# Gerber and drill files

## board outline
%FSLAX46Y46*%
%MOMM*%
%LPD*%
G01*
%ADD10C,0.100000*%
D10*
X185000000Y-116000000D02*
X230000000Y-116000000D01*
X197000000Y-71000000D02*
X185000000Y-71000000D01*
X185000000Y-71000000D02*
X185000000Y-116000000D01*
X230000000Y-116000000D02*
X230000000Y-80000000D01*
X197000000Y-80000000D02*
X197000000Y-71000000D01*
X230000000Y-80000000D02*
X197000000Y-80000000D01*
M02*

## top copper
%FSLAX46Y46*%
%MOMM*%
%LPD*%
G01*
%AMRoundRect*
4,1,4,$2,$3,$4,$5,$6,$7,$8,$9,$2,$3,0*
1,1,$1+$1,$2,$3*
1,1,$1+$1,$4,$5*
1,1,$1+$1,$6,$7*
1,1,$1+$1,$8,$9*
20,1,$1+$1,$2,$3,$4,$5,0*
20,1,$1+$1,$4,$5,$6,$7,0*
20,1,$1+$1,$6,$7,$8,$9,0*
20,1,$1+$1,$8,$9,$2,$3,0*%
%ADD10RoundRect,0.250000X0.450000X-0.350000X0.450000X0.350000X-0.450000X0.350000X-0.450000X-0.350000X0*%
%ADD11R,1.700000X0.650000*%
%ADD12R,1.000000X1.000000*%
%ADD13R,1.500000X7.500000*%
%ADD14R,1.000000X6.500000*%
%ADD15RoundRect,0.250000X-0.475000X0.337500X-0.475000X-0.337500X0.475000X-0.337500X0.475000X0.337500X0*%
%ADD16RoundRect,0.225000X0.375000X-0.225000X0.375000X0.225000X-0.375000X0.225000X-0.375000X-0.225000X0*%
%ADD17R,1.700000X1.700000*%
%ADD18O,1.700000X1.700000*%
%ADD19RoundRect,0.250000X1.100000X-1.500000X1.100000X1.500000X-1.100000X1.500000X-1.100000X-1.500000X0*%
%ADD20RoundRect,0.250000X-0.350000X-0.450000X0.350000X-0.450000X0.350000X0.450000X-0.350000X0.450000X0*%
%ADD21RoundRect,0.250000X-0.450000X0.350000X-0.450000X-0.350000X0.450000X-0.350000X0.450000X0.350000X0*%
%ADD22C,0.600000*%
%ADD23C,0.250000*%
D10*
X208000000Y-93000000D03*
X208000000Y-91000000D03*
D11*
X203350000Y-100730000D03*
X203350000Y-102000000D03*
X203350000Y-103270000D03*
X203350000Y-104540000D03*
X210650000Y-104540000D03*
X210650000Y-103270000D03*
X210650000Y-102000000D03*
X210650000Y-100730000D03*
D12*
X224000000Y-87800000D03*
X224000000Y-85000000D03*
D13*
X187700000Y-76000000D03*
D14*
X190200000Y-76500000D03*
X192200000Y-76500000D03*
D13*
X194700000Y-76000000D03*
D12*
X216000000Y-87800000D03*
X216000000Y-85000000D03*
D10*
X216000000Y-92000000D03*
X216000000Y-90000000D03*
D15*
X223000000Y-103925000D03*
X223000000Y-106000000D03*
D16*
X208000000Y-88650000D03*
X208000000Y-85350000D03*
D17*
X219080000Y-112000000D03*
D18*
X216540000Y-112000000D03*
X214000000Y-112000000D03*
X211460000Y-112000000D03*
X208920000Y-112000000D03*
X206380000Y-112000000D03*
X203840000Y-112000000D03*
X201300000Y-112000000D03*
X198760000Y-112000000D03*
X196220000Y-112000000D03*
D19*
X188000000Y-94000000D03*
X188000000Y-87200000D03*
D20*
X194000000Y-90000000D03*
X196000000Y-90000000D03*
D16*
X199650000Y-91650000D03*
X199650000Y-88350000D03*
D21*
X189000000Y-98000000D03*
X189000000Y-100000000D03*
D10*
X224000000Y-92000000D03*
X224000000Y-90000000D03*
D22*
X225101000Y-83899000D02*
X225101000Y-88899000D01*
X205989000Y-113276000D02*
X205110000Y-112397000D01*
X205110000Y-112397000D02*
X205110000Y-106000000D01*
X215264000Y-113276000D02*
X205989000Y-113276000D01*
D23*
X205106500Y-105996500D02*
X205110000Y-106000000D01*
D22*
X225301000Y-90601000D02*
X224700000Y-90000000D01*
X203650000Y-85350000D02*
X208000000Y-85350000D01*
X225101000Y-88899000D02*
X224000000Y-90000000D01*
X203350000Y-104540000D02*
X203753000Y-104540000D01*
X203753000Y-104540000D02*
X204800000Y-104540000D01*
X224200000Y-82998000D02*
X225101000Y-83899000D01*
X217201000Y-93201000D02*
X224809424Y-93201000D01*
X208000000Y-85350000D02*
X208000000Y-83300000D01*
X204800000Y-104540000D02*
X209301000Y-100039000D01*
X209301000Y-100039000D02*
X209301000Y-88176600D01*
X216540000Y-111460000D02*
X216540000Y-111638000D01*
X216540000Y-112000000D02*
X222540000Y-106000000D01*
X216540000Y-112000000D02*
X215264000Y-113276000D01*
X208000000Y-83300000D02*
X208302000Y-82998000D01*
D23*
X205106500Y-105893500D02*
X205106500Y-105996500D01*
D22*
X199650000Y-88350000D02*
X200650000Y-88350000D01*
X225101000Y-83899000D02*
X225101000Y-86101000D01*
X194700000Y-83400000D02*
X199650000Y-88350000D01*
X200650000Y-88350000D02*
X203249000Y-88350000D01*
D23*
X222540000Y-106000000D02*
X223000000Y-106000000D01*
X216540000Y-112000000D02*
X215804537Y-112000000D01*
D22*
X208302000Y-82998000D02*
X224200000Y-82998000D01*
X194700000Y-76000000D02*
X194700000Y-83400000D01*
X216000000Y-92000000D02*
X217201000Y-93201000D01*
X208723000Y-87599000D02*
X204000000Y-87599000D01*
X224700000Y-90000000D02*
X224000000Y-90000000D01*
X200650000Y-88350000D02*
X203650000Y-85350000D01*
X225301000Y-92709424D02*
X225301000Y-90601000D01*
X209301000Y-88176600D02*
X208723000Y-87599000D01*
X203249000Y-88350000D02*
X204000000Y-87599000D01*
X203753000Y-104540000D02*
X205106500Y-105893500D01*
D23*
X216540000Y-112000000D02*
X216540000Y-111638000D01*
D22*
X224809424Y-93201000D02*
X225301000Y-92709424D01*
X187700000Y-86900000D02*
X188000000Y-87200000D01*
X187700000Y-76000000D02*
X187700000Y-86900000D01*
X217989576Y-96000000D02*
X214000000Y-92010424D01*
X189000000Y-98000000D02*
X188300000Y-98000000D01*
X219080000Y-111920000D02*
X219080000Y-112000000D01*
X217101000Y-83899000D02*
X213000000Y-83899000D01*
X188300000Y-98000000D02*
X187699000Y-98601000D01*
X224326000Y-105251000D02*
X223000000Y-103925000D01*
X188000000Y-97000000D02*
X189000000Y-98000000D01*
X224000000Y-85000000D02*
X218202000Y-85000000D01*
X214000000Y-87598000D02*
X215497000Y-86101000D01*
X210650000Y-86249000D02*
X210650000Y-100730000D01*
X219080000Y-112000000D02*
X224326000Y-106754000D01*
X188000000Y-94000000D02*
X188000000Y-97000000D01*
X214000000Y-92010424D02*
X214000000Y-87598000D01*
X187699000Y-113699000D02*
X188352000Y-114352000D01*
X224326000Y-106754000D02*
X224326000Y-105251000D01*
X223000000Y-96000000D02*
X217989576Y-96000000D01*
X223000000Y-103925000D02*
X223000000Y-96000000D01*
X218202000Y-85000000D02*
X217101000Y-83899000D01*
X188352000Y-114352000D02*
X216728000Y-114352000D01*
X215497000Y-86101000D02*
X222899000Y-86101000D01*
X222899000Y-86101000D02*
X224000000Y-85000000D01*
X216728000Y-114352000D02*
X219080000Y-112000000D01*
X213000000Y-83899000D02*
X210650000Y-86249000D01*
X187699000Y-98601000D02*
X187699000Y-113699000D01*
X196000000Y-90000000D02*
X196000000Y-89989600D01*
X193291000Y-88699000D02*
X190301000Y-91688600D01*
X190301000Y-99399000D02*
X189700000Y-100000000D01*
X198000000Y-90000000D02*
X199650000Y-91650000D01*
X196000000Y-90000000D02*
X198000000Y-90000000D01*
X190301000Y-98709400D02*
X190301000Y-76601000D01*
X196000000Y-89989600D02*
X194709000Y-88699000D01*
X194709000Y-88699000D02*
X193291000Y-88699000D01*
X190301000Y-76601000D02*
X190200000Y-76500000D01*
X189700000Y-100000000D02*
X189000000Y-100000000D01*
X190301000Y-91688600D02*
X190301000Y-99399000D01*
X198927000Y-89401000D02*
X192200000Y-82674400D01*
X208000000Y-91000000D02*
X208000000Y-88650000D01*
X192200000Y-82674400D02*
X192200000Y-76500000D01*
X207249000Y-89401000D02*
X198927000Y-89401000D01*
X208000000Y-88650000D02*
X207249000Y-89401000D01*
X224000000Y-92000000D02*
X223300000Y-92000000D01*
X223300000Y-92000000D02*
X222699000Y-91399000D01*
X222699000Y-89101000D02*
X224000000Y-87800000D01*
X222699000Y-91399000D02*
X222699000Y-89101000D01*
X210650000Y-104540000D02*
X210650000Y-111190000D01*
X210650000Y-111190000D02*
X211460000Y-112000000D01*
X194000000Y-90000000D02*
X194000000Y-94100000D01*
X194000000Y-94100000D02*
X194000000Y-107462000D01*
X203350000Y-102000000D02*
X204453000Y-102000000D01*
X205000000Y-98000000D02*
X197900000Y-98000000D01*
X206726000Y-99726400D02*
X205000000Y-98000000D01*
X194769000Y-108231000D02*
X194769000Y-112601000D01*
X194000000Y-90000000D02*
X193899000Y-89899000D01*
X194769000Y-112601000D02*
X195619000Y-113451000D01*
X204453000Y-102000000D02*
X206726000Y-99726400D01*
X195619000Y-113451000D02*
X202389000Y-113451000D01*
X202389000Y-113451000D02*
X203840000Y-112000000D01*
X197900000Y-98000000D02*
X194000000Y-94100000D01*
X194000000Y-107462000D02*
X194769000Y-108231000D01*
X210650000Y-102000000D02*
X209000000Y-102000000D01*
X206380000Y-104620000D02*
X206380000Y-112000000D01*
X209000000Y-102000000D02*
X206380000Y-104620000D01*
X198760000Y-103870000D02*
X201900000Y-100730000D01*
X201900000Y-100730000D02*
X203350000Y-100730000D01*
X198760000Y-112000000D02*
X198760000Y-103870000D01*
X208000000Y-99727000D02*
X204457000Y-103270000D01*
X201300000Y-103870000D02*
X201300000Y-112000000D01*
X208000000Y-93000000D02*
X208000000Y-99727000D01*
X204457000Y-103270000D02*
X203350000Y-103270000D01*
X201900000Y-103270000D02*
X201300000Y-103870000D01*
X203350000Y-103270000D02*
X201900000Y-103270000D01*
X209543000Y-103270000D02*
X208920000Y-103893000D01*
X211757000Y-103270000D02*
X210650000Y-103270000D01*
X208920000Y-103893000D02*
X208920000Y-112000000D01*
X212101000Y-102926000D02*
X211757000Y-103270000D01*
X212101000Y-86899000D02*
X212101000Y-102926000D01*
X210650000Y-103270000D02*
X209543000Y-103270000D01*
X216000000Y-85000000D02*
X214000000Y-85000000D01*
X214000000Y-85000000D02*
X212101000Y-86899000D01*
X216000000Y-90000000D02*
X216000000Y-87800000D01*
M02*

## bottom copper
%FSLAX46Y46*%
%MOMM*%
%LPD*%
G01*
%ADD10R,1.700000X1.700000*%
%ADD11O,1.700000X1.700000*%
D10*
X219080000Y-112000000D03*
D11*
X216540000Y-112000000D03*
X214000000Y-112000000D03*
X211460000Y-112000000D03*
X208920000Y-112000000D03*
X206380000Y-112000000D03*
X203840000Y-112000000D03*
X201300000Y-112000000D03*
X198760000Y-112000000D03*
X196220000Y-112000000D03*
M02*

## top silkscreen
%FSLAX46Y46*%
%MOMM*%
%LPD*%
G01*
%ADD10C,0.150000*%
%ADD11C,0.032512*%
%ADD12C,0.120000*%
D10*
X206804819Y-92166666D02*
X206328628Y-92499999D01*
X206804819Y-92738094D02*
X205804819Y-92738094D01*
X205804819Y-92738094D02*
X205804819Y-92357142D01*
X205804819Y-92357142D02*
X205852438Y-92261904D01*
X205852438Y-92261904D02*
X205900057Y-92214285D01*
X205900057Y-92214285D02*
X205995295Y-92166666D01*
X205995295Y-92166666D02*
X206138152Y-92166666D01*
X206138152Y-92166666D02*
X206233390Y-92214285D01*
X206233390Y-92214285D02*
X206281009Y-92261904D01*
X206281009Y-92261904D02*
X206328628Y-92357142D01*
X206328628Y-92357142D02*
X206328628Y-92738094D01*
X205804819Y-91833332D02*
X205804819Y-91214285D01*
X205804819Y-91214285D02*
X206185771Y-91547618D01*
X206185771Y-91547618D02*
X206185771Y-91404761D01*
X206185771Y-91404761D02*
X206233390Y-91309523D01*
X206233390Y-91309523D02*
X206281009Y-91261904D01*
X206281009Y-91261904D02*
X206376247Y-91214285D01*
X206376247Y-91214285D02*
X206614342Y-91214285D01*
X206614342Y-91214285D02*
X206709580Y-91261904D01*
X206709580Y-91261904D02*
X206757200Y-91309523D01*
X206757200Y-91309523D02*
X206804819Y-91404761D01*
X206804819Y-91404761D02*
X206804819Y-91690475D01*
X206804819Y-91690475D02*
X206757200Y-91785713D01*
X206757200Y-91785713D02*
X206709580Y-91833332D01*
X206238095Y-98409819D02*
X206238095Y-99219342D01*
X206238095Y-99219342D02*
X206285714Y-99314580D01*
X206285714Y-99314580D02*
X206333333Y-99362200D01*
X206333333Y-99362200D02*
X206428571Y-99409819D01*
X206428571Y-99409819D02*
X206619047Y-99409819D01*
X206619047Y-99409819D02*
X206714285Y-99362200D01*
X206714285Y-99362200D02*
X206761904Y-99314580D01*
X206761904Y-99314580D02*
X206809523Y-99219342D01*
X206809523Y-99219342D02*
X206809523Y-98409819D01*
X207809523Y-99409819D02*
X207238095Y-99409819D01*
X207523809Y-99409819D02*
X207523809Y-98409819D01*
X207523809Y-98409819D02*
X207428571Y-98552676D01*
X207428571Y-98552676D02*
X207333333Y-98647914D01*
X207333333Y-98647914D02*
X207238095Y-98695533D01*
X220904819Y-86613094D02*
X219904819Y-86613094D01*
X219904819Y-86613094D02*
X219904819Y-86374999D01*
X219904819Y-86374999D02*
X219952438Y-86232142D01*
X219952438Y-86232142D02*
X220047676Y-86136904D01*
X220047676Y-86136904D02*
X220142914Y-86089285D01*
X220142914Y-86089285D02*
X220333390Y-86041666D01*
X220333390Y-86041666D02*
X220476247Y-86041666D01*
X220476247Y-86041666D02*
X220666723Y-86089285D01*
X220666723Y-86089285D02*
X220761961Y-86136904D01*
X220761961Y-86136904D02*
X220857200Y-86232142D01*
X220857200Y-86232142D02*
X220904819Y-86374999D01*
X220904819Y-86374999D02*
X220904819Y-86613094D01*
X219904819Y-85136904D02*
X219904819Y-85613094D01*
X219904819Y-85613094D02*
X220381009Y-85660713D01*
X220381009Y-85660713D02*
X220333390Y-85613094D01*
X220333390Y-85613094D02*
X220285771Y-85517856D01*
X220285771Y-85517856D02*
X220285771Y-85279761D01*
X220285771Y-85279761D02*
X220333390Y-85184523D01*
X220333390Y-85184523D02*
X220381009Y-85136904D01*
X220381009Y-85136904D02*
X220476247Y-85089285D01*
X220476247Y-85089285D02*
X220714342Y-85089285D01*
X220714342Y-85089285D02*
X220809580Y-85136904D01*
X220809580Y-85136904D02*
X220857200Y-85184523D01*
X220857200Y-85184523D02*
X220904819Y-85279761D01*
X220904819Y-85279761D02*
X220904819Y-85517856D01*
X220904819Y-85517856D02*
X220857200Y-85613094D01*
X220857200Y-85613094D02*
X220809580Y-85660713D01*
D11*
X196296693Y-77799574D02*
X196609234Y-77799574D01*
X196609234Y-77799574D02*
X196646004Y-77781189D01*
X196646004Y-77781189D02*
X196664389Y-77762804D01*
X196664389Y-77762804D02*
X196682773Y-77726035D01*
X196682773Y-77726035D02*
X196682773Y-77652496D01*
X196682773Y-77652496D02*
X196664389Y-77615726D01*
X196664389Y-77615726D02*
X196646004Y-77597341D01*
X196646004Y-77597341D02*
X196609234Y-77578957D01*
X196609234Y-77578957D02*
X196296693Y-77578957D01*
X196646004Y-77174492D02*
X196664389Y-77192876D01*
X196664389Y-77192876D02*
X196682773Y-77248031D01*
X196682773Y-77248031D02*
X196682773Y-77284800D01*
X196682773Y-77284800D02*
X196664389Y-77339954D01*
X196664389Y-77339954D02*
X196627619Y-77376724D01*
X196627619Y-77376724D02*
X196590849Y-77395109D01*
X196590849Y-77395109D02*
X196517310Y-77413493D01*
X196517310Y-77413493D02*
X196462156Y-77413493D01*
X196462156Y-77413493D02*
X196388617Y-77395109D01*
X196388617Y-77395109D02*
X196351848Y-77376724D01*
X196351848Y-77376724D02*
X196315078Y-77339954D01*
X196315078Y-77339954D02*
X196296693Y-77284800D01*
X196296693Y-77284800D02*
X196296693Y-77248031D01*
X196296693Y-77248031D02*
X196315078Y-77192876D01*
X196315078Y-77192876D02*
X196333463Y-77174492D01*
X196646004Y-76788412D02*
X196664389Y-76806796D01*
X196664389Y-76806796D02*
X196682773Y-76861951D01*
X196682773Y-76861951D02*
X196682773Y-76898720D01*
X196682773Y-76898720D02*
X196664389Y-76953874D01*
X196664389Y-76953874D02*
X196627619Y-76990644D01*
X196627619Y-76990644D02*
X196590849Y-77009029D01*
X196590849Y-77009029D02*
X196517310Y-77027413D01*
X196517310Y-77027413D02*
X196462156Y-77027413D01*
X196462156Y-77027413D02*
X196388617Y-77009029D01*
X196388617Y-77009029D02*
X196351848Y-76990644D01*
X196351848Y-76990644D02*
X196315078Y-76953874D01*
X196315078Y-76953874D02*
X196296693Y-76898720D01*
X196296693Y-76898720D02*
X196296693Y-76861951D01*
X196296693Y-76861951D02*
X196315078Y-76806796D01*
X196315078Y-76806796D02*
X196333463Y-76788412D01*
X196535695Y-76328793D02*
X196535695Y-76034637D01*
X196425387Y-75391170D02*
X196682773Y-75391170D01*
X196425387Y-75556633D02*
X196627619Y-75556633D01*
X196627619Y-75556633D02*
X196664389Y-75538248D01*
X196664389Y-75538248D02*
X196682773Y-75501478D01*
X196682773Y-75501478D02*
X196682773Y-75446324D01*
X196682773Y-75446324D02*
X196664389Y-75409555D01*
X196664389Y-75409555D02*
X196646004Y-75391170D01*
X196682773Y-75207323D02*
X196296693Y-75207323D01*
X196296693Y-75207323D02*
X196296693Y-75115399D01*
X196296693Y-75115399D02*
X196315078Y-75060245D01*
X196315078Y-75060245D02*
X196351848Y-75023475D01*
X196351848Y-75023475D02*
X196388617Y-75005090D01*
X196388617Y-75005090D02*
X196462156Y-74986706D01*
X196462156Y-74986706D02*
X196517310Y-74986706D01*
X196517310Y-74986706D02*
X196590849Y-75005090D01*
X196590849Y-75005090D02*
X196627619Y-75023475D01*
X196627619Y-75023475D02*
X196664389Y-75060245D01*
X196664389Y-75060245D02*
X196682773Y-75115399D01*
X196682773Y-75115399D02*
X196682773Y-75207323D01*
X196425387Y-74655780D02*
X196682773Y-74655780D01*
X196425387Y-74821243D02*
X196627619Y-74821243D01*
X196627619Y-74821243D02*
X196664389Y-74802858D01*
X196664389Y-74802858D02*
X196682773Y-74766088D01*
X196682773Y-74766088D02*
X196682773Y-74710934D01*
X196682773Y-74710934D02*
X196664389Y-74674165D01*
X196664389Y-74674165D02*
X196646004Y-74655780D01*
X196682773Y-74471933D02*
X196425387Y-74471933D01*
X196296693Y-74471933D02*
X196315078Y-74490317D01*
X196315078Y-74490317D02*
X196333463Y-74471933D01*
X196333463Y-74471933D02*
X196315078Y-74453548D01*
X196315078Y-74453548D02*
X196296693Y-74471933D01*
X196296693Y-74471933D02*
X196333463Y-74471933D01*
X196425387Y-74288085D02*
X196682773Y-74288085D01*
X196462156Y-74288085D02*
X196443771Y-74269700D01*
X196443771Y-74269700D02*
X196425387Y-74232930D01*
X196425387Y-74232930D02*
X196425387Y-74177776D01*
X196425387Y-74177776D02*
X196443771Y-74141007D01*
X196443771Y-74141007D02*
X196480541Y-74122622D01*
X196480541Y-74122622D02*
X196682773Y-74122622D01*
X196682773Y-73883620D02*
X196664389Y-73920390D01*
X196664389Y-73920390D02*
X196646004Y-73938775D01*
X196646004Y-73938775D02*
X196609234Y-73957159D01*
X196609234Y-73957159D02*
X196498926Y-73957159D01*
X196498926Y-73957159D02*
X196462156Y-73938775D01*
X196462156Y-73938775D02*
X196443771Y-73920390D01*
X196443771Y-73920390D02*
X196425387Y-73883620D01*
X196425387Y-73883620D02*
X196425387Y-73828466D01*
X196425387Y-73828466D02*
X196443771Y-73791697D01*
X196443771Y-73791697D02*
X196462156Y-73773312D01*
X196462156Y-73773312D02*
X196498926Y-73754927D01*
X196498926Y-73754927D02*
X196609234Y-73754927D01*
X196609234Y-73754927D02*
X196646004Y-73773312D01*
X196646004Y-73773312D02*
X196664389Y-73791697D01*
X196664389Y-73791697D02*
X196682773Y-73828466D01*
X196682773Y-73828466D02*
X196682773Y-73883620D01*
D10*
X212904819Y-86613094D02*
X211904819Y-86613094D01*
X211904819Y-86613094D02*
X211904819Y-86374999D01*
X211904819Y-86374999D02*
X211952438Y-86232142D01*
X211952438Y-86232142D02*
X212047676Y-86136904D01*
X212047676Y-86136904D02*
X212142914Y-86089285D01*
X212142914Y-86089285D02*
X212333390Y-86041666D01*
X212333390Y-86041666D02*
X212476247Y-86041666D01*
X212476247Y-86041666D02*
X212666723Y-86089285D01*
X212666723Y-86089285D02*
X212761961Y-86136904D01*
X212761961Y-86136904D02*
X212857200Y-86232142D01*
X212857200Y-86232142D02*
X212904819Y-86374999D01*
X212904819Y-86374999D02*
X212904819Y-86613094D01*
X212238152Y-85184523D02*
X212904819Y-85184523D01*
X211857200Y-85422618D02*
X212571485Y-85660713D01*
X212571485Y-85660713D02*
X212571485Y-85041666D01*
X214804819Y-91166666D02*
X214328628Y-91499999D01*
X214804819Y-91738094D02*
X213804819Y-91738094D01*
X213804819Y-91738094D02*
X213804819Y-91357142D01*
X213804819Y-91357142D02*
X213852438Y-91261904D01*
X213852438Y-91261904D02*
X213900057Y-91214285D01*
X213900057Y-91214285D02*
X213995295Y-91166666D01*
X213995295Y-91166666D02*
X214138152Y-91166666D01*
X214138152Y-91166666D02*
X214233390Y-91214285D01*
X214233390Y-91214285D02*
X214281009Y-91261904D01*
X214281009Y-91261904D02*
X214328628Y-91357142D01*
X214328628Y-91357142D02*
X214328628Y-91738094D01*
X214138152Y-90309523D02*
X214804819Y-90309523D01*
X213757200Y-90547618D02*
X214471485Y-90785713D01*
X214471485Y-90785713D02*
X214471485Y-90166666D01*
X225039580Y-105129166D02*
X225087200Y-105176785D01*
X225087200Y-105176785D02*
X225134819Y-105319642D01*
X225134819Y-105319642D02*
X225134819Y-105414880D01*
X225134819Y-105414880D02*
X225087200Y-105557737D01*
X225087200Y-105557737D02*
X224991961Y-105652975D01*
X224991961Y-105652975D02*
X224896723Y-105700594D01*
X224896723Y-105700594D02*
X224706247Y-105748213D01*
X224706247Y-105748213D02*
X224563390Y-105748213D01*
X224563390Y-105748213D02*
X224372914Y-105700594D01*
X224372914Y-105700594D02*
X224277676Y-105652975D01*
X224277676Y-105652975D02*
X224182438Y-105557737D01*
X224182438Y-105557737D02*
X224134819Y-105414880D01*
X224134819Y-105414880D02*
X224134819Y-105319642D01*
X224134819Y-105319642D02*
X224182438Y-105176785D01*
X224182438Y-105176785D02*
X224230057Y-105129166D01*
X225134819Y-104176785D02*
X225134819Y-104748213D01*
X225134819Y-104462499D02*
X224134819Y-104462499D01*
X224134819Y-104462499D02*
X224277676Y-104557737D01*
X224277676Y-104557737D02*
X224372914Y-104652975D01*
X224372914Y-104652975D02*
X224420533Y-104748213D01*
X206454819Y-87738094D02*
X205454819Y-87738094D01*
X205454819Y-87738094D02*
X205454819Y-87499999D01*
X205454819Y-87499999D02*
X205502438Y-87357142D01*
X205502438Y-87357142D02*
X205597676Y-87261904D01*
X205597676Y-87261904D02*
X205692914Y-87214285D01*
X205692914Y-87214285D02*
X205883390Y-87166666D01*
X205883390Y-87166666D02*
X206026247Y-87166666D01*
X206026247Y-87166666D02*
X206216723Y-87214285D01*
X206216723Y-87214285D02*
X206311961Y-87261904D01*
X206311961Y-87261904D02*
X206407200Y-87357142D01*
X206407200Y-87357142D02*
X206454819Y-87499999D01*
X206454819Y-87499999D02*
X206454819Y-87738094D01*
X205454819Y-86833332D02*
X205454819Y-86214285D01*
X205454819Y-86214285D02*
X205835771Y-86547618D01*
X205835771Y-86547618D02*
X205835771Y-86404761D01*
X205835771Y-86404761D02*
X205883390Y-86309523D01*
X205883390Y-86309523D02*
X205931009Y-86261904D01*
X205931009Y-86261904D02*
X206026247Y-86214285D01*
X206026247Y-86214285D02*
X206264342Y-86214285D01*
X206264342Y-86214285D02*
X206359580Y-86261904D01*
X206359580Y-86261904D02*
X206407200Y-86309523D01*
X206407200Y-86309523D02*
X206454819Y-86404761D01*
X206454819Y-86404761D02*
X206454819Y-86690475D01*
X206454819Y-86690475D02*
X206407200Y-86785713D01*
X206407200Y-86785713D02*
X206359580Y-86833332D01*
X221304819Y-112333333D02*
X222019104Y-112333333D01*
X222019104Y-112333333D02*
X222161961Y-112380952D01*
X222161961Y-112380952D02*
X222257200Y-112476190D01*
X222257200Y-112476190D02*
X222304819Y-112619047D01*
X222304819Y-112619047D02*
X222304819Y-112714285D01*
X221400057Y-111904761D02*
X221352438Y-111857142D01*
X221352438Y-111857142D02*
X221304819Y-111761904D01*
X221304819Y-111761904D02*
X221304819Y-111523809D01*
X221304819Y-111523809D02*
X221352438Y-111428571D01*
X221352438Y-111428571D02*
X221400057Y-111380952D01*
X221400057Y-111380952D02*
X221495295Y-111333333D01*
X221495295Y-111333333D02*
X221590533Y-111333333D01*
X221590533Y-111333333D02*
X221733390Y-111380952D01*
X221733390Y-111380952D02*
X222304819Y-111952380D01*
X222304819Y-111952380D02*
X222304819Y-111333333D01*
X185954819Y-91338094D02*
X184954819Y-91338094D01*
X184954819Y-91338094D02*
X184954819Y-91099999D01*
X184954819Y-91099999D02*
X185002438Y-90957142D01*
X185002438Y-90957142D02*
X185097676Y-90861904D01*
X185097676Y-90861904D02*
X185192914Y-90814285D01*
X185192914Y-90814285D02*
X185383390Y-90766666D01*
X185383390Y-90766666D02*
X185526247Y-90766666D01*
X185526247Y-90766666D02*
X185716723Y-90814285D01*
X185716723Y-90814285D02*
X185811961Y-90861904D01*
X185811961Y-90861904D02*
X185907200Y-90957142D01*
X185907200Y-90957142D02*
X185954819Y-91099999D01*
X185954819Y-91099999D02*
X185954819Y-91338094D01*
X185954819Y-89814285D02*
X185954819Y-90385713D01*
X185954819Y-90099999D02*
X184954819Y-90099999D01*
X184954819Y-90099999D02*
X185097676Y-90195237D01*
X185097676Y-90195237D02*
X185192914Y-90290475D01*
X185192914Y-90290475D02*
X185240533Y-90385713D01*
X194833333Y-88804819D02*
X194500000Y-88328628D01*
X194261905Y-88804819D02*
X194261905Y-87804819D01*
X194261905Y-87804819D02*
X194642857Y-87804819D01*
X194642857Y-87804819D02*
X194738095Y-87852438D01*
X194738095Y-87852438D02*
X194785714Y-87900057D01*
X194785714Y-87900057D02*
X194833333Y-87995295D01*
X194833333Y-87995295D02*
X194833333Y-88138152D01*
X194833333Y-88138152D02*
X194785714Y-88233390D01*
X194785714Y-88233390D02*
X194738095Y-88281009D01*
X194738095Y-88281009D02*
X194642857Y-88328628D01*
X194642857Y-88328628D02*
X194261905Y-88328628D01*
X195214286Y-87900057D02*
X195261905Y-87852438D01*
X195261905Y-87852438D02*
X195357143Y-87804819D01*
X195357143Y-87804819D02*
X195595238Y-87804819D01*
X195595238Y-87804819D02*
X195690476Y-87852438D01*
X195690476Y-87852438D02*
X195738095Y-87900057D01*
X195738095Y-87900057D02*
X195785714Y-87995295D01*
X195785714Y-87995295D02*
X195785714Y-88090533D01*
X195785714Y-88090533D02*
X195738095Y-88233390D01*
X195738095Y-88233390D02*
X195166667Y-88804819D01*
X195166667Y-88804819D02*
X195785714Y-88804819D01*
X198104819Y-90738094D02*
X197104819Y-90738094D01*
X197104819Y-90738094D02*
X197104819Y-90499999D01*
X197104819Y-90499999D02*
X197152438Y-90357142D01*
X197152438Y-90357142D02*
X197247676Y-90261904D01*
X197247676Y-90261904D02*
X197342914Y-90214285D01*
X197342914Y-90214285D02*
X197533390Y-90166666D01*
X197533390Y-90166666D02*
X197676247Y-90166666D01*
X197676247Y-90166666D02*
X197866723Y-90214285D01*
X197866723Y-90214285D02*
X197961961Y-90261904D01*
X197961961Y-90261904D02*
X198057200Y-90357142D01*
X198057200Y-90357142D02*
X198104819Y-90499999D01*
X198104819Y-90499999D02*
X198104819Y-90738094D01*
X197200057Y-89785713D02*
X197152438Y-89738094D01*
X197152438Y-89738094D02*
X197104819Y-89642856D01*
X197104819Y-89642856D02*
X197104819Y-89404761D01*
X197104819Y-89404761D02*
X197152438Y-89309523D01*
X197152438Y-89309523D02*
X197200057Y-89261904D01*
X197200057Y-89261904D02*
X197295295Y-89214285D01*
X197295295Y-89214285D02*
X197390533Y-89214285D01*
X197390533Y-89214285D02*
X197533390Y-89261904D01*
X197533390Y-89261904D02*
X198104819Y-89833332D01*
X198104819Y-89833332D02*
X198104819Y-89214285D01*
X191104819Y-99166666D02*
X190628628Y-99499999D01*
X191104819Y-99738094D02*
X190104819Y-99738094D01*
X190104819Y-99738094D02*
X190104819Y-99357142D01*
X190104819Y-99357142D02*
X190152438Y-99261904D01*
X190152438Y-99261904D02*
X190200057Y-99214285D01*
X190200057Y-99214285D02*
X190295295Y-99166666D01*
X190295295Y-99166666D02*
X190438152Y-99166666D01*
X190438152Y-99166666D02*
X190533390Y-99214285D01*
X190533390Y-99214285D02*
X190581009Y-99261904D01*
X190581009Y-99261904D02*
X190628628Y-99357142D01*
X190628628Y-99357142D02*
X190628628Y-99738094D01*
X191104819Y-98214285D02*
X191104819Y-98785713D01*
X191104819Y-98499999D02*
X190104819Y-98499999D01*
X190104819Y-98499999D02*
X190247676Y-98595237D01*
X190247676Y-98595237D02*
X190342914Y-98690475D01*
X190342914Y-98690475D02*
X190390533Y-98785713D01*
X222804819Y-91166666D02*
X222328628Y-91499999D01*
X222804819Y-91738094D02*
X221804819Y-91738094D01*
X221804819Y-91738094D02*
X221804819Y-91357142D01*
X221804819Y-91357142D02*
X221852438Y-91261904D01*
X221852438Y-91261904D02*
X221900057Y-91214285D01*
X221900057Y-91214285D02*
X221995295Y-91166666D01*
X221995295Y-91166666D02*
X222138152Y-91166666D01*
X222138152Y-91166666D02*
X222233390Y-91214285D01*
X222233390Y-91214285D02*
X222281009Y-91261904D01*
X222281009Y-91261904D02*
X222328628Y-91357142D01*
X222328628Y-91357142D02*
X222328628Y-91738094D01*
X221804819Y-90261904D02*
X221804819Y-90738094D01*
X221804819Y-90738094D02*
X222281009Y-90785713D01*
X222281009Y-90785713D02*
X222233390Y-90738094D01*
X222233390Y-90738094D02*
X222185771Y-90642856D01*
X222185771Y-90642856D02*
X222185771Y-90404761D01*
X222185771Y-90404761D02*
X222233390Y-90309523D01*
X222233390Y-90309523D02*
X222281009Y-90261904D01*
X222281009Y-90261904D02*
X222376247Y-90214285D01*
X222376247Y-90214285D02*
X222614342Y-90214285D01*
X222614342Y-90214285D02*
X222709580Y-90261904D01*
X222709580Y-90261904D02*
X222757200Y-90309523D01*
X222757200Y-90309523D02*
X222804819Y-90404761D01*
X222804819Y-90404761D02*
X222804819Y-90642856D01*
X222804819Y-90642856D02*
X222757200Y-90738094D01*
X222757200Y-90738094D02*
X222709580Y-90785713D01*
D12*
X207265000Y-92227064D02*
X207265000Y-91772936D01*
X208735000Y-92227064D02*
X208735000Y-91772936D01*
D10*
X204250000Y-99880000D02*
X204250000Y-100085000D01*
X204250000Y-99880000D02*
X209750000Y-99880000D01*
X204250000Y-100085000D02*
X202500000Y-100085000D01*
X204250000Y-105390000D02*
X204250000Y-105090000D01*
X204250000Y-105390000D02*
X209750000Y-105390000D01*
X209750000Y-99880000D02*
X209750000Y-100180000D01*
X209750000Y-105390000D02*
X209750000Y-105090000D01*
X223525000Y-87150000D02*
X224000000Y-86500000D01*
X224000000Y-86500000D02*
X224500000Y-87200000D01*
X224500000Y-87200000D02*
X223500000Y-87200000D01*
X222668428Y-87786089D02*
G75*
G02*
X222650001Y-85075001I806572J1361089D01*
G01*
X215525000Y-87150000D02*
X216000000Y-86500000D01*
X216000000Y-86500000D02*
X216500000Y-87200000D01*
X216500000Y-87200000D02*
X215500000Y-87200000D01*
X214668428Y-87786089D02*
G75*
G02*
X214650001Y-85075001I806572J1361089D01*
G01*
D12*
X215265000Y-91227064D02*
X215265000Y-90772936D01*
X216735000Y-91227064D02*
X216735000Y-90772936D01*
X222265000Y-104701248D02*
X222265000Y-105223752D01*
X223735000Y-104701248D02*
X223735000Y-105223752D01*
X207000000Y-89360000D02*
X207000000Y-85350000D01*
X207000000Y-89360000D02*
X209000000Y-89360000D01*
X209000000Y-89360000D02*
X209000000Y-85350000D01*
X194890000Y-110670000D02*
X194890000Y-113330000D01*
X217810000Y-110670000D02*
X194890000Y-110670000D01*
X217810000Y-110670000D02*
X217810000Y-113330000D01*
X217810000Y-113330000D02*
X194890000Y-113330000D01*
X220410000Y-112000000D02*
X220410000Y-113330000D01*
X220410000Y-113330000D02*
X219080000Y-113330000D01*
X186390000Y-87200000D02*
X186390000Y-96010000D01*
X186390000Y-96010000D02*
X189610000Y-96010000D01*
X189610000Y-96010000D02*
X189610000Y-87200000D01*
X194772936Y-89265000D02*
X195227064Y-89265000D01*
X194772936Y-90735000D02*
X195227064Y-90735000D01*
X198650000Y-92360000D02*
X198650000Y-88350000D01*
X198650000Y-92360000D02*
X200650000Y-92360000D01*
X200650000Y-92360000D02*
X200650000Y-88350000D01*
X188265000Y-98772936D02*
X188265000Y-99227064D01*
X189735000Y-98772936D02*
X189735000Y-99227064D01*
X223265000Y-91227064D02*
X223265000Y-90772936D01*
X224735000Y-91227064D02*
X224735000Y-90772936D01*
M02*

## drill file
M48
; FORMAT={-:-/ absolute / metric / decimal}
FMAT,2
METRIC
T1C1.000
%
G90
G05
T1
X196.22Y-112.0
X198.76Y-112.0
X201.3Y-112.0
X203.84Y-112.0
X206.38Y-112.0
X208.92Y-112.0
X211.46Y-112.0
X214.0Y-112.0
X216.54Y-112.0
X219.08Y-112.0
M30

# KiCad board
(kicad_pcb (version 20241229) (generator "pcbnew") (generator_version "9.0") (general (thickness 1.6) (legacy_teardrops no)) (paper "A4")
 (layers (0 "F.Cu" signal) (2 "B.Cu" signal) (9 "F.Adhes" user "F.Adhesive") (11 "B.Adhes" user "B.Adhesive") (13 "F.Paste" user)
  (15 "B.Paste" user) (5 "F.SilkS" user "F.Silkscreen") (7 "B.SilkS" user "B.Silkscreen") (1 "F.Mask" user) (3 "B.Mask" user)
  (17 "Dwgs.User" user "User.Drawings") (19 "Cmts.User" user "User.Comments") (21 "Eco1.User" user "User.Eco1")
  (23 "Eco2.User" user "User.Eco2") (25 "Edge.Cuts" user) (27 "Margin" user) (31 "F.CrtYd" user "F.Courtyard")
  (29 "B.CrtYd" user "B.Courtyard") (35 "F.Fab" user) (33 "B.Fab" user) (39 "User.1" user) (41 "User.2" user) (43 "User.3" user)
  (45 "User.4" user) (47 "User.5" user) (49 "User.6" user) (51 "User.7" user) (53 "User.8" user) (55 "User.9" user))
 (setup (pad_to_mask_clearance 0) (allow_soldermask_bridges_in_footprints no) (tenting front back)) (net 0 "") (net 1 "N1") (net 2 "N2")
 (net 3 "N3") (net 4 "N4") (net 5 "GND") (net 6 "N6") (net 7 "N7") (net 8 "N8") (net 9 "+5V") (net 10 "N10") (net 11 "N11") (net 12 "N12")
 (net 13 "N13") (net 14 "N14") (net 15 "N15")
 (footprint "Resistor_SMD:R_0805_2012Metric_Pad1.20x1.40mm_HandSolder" (layer "F.Cu") (at 208 92 90)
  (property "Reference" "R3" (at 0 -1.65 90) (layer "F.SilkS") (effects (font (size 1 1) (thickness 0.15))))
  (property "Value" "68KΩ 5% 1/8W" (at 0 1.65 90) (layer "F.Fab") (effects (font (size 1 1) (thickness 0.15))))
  (fp_line (start -0.227064 -0.735) (end 0.227064 -0.735) (stroke (width 0.12) (type solid)) (layer "F.SilkS"))
  (fp_line (start -0.227064 0.735) (end 0.227064 0.735) (stroke (width 0.12) (type solid)) (layer "F.SilkS"))
  (pad "1" smd roundrect (at -1 0 90) (size 1.2 1.4) (layers "F.Cu" "F.Mask" "F.Paste") (roundrect_rratio 0.208333) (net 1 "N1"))
  (pad "2" smd roundrect (at 1 0 90) (size 1.2 1.4) (layers "F.Cu" "F.Mask" "F.Paste") (roundrect_rratio 0.208333) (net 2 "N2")))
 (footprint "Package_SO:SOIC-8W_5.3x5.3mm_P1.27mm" (layer "F.Cu") (at 207 102.635)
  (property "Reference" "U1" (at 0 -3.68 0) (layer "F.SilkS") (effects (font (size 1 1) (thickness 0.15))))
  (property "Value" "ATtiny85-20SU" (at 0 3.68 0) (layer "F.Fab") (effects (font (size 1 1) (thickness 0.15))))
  (fp_line (start -2.75 -2.755) (end -2.75 -2.55) (stroke (width 0.15) (type solid)) (layer "F.SilkS"))
  (fp_line (start -2.75 -2.755) (end 2.75 -2.755) (stroke (width 0.15) (type solid)) (layer "F.SilkS"))
  (fp_line (start -2.75 -2.55) (end -4.5 -2.55) (stroke (width 0.15) (type solid)) (layer "F.SilkS"))
  (fp_line (start -2.75 2.755) (end -2.75 2.455) (stroke (width 0.15) (type solid)) (layer "F.SilkS"))
  (fp_line (start -2.75 2.755) (end 2.75 2.755) (stroke (width 0.15) (type solid)) (layer "F.SilkS"))
  (fp_line (start 2.75 -2.755) (end 2.75 -2.455) (stroke (width 0.15) (type solid)) (layer "F.SilkS"))
  (fp_line (start 2.75 2.755) (end 2.75 2.455) (stroke (width 0.15) (type solid)) (layer "F.SilkS"))
  (pad "1" smd rect (at -3.65 -1.905) (size 1.7 0.65) (layers "F.Cu" "F.Mask" "F.Paste") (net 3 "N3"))
  (pad "2" smd rect (at -3.65 -0.635) (size 1.7 0.65) (layers "F.Cu" "F.Mask" "F.Paste") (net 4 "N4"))
  (pad "3" smd rect (at -3.65 0.635) (size 1.7 0.65) (layers "F.Cu" "F.Mask" "F.Paste") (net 1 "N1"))
  (pad "4" smd rect (at -3.65 1.905) (size 1.7 0.65) (layers "F.Cu" "F.Mask" "F.Paste") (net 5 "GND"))
  (pad "5" smd rect (at 3.65 1.905) (size 1.7 0.65) (layers "F.Cu" "F.Mask" "F.Paste") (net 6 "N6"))
  (pad "6" smd rect (at 3.65 0.635) (size 1.7 0.65) (layers "F.Cu" "F.Mask" "F.Paste") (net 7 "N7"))
  (pad "7" smd rect (at 3.65 -0.635) (size 1.7 0.65) (layers "F.Cu" "F.Mask" "F.Paste") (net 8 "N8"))
  (pad "8" smd rect (at 3.65 -1.905) (size 1.7 0.65) (layers "F.Cu" "F.Mask" "F.Paste") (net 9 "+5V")))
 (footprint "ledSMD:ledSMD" (layer "F.Cu") (at 224 86 90)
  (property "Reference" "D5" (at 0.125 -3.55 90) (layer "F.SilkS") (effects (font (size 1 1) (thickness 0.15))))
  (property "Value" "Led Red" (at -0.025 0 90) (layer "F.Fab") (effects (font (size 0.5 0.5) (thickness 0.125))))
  (fp_line (start -1.15 -0.475) (end -0.5 0) (stroke (width 0.15) (type solid)) (layer "F.SilkS"))
  (fp_line (start -0.5 0) (end -1.2 0.5) (stroke (width 0.15) (type solid)) (layer "F.SilkS"))
  (fp_line (start -1.2 0.5) (end -1.2 -0.5) (stroke (width 0.15) (type solid)) (layer "F.SilkS"))
  (fp_arc (start -1.786089 -1.331572) (mid -0.435753 -2.107089) (end 0.924999 -1.349999) (stroke (width 0.15) (type solid))
   (layer "F.SilkS"))
  (pad "1" smd rect (at -1.8 0 90) (size 1 1) (layers "F.Cu" "F.Mask" "F.Paste") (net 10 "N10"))
  (pad "2" smd rect (at 1 0 90) (size 1 1) (layers "F.Cu" "F.Mask" "F.Paste") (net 9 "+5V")))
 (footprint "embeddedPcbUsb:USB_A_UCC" (layer "F.Cu") (at 191.2 76.2 -90)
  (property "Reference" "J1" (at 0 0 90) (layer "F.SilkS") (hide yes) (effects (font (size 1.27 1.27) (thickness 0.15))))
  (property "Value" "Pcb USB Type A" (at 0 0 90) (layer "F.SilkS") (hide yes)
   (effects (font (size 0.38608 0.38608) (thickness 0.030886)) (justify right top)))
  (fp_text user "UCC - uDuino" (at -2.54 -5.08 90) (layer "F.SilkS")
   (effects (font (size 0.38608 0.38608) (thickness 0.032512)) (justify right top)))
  (pad "1" smd rect (at -0.2 3.5 270) (size 7.5 1.5) (layers "F.Cu" "F.Mask" "F.Paste") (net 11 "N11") (solder_mask_margin 0.1016))
  (pad "2" smd rect (at 0.3 1 270) (size 6.5 1) (layers "F.Cu" "F.Mask" "F.Paste") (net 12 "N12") (solder_mask_margin 0.1016))
  (pad "3" smd rect (at 0.3 -1 270) (size 6.5 1) (layers "F.Cu" "F.Mask" "F.Paste") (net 2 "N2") (solder_mask_margin 0.1016))
  (pad "4" smd rect (at -0.2 -3.5 270) (size 7.5 1.5) (layers "F.Cu" "F.Mask" "F.Paste") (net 5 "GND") (solder_mask_margin 0.1016)))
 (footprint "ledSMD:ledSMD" (layer "F.Cu") (at 216 86 90)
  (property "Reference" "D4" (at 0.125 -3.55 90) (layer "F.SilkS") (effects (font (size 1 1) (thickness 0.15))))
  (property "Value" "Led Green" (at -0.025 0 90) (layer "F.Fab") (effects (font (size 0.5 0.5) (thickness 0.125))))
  (fp_line (start -1.15 -0.475) (end -0.5 0) (stroke (width 0.15) (type solid)) (layer "F.SilkS"))
  (fp_line (start -0.5 0) (end -1.2 0.5) (stroke (width 0.15) (type solid)) (layer "F.SilkS"))
  (fp_line (start -1.2 0.5) (end -1.2 -0.5) (stroke (width 0.15) (type solid)) (layer "F.SilkS"))
  (fp_arc (start -1.786089 -1.331572) (mid -0.435753 -2.107089) (end 0.924999 -1.349999) (stroke (width 0.15) (type solid))
   (layer "F.SilkS"))
  (pad "1" smd rect (at -1.8 0 90) (size 1 1) (layers "F.Cu" "F.Mask" "F.Paste") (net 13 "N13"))
  (pad "2" smd rect (at 1 0 90) (size 1 1) (layers "F.Cu" "F.Mask" "F.Paste") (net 7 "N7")))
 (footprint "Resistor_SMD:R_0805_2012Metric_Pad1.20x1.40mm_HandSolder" (layer "F.Cu") (at 216 91 90)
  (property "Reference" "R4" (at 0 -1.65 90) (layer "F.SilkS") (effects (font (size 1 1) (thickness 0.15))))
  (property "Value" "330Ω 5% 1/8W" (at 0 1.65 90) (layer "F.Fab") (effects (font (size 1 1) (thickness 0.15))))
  (fp_line (start -0.227064 -0.735) (end 0.227064 -0.735) (stroke (width 0.12) (type solid)) (layer "F.SilkS"))
  (fp_line (start -0.227064 0.735) (end 0.227064 0.735) (stroke (width 0.12) (type solid)) (layer "F.SilkS"))
  (pad "1" smd roundrect (at -1 0 90) (size 1.2 1.4) (layers "F.Cu" "F.Mask" "F.Paste") (roundrect_rratio 0.208333) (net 5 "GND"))
  (pad "2" smd roundrect (at 1 0 90) (size 1.2 1.4) (layers "F.Cu" "F.Mask" "F.Paste") (roundrect_rratio 0.208333) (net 13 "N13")))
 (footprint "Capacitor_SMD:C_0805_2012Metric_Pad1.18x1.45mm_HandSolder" (layer "F.Cu") (at 223 104.9625 -90)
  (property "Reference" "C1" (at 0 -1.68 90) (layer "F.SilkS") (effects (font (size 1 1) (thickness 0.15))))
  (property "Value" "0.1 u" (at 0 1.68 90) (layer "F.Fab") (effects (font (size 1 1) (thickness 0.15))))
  (fp_line (start -0.261252 0.735) (end 0.261252 0.735) (stroke (width 0.12) (type solid)) (layer "F.SilkS"))
  (fp_line (start -0.261252 -0.735) (end 0.261252 -0.735) (stroke (width 0.12) (type solid)) (layer "F.SilkS"))
  (pad "1" smd roundrect (at -1.0375 0 270) (size 1.175 1.45) (layers "F.Cu" "F.Mask" "F.Paste") (roundrect_rratio 0.212766) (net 9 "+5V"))
  (pad "2" smd roundrect (at 1.0375 0 270) (size 1.175 1.45) (layers "F.Cu" "F.Mask" "F.Paste") (roundrect_rratio 0.212766) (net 5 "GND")))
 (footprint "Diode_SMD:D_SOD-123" (layer "F.Cu") (at 208 87 90)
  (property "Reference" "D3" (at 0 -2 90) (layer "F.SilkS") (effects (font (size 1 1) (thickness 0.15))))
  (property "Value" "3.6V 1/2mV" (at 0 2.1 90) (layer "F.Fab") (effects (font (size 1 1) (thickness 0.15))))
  (fp_line (start -2.36 -1) (end 1.65 -1) (stroke (width 0.12) (type solid)) (layer "F.SilkS"))
  (fp_line (start -2.36 -1) (end -2.36 1) (stroke (width 0.12) (type solid)) (layer "F.SilkS"))
  (fp_line (start -2.36 1) (end 1.65 1) (stroke (width 0.12) (type solid)) (layer "F.SilkS"))
  (pad "1" smd roundrect (at -1.65 0 90) (size 0.9 1.2) (layers "F.Cu" "F.Mask" "F.Paste") (roundrect_rratio 0.25) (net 2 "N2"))
  (pad "2" smd roundrect (at 1.65 0 90) (size 0.9 1.2) (layers "F.Cu" "F.Mask" "F.Paste") (roundrect_rratio 0.25) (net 5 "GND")))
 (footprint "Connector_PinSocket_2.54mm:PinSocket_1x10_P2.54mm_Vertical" (layer "F.Cu") (at 219.08 112 -90)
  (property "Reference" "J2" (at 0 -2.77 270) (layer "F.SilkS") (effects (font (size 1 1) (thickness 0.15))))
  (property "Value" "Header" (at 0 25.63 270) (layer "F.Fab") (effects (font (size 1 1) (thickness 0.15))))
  (fp_line (start -1.33 24.19) (end 1.33 24.19) (stroke (width 0.12) (type solid)) (layer "F.SilkS"))
  (fp_line (start -1.33 1.27) (end -1.33 24.19) (stroke (width 0.12) (type solid)) (layer "F.SilkS"))
  (fp_line (start -1.33 1.27) (end 1.33 1.27) (stroke (width 0.12) (type solid)) (layer "F.SilkS"))
  (fp_line (start 1.33 1.27) (end 1.33 24.19) (stroke (width 0.12) (type solid)) (layer "F.SilkS"))
  (fp_line (start 0 -1.33) (end 1.33 -1.33) (stroke (width 0.12) (type solid)) (layer "F.SilkS"))
  (fp_line (start 1.33 -1.33) (end 1.33 0) (stroke (width 0.12) (type solid)) (layer "F.SilkS"))
  (pad "1" thru_hole rect (at 0 0 270) (size 1.7 1.7) (drill 1) (layers "*.Cu" "*.Mask") (remove_unused_layers no) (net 9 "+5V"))
  (pad "2" thru_hole oval (at 0 2.54 270) (size 1.7 1.7) (drill 1) (layers "*.Cu" "*.Mask") (remove_unused_layers no) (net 5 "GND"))
  (pad "3" thru_hole oval (at 0 5.08 270) (size 1.7 1.7) (drill 1) (layers "*.Cu" "*.Mask") (remove_unused_layers no) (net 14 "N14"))
  (pad "4" thru_hole oval (at 0 7.62 270) (size 1.7 1.7) (drill 1) (layers "*.Cu" "*.Mask") (remove_unused_layers no) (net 6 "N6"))
  (pad "5" thru_hole oval (at 0 10.16 270) (size 1.7 1.7) (drill 1) (layers "*.Cu" "*.Mask") (remove_unused_layers no) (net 7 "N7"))
  (pad "6" thru_hole oval (at 0 12.7 270) (size 1.7 1.7) (drill 1) (layers "*.Cu" "*.Mask") (remove_unused_layers no) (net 8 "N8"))
  (pad "7" thru_hole oval (at 0 15.24 270) (size 1.7 1.7) (drill 1) (layers "*.Cu" "*.Mask") (remove_unused_layers no) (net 4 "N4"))
  (pad "8" thru_hole oval (at 0 17.78 270) (size 1.7 1.7) (drill 1) (layers "*.Cu" "*.Mask") (remove_unused_layers no) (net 1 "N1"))
  (pad "9" thru_hole oval (at 0 20.32 270) (size 1.7 1.7) (drill 1) (layers "*.Cu" "*.Mask") (remove_unused_layers no) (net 3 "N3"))
  (pad "10" thru_hole oval (at 0 22.86 270) (size 1.7 1.7) (drill 1) (layers "*.Cu" "*.Mask") (remove_unused_layers no) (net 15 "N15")))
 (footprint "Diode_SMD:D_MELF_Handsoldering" (layer "F.Cu") (at 188 90.6 90)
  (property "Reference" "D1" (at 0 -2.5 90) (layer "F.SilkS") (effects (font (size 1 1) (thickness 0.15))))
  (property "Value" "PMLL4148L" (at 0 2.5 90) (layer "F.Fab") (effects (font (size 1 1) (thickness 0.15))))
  (fp_line (start 3.4 -1.61) (end -5.41 -1.61) (stroke (width 0.12) (type solid)) (layer "F.SilkS"))
  (fp_line (start -5.41 -1.61) (end -5.41 1.61) (stroke (width 0.12) (type solid)) (layer "F.SilkS"))
  (fp_line (start -5.41 1.61) (end 3.4 1.61) (stroke (width 0.12) (type solid)) (layer "F.SilkS"))
  (pad "1" smd roundrect (at -3.4 0 90) (size 3.5 2.7) (layers "F.Cu" "F.Mask" "F.Paste") (roundrect_rratio 0.0925925926) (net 9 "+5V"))
  (pad "2" smd roundrect (at 3.4 0 90) (size 3.5 2.7) (layers "F.Cu" "F.Mask" "F.Paste") (roundrect_rratio 0.0925925926) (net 11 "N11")))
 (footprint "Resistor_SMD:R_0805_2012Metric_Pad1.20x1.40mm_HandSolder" (layer "F.Cu") (at 195 90)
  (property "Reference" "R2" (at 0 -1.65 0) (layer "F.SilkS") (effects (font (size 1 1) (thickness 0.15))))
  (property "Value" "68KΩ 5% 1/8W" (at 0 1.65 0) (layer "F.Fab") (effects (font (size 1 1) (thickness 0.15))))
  (fp_line (start -0.227064 -0.735) (end 0.227064 -0.735) (stroke (width 0.12) (type solid)) (layer "F.SilkS"))
  (fp_line (start -0.227064 0.735) (end 0.227064 0.735) (stroke (width 0.12) (type solid)) (layer "F.SilkS"))
  (pad "1" smd roundrect (at -1 0) (size 1.2 1.4) (layers "F.Cu" "F.Mask" "F.Paste") (roundrect_rratio 0.208333) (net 4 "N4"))
  (pad "2" smd roundrect (at 1 0) (size 1.2 1.4) (layers "F.Cu" "F.Mask" "F.Paste") (roundrect_rratio 0.208333) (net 12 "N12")))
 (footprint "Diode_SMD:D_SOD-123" (layer "F.Cu") (at 199.65 90 90)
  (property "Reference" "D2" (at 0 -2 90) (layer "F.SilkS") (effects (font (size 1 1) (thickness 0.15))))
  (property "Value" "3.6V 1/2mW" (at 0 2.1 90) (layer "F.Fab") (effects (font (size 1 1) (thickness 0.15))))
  (fp_line (start -2.36 -1) (end 1.65 -1) (stroke (width 0.12) (type solid)) (layer "F.SilkS"))
  (fp_line (start -2.36 -1) (end -2.36 1) (stroke (width 0.12) (type solid)) (layer "F.SilkS"))
  (fp_line (start -2.36 1) (end 1.65 1) (stroke (width 0.12) (type solid)) (layer "F.SilkS"))
  (pad "1" smd roundrect (at -1.65 0 90) (size 0.9 1.2) (layers "F.Cu" "F.Mask" "F.Paste") (roundrect_rratio 0.25) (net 12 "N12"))
  (pad "2" smd roundrect (at 1.65 0 90) (size 0.9 1.2) (layers "F.Cu" "F.Mask" "F.Paste") (roundrect_rratio 0.25) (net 5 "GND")))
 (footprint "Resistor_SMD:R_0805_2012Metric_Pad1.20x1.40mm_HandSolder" (layer "F.Cu") (at 189 99 -90)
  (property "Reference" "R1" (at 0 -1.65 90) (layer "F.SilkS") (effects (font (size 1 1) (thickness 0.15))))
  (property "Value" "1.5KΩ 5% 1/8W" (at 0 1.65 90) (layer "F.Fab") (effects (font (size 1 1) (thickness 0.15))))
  (fp_line (start -0.227064 0.735) (end 0.227064 0.735) (stroke (width 0.12) (type solid)) (layer "F.SilkS"))
  (fp_line (start -0.227064 -0.735) (end 0.227064 -0.735) (stroke (width 0.12) (type solid)) (layer "F.SilkS"))
  (pad "1" smd roundrect (at -1 0 270) (size 1.2 1.4) (layers "F.Cu" "F.Mask" "F.Paste") (roundrect_rratio 0.208333) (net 9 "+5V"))
  (pad "2" smd roundrect (at 1 0 270) (size 1.2 1.4) (layers "F.Cu" "F.Mask" "F.Paste") (roundrect_rratio 0.208333) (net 12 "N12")))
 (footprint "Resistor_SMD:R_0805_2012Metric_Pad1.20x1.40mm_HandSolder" (layer "F.Cu") (at 224 91 90)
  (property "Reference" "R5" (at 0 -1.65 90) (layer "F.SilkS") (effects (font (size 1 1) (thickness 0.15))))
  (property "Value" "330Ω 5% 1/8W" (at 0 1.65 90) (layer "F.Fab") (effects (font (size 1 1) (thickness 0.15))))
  (fp_line (start -0.227064 -0.735) (end 0.227064 -0.735) (stroke (width 0.12) (type solid)) (layer "F.SilkS"))
  (fp_line (start -0.227064 0.735) (end 0.227064 0.735) (stroke (width 0.12) (type solid)) (layer "F.SilkS"))
  (pad "1" smd roundrect (at -1 0 90) (size 1.2 1.4) (layers "F.Cu" "F.Mask" "F.Paste") (roundrect_rratio 0.208333) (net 10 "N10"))
  (pad "2" smd roundrect (at 1 0 90) (size 1.2 1.4) (layers "F.Cu" "F.Mask" "F.Paste") (roundrect_rratio 0.208333) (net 5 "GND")))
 (gr_line (start 185 116) (end 230 116) (stroke (width 0.1) (type default)) (layer "Edge.Cuts"))
 (gr_line (start 197 71) (end 185 71) (stroke (width 0.1) (type default)) (layer "Edge.Cuts"))
 (gr_line (start 185 71) (end 185 116) (stroke (width 0.1) (type default)) (layer "Edge.Cuts"))
 (gr_line (start 230 116) (end 230 80) (stroke (width 0.1) (type default)) (layer "Edge.Cuts"))
 (gr_line (start 197 80) (end 197 71) (stroke (width 0.1) (type default)) (layer "Edge.Cuts"))
 (gr_line (start 230 80) (end 197 80) (stroke (width 0.1) (type default)) (layer "Edge.Cuts"))
 (segment (start 225.101 83.899) (end 225.101 88.899) (width 0.6) (layer "F.Cu") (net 5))
 (segment (start 205.989 113.276) (end 205.11 112.397) (width 0.6) (layer "F.Cu") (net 5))
 (segment (start 205.11 112.397) (end 205.11 106) (width 0.6) (layer "F.Cu") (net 5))
 (segment (start 215.264 113.276) (end 205.989 113.276) (width 0.6) (layer "F.Cu") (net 5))
 (segment (start 205.1065 105.9965) (end 205.11 106) (width 0.25) (layer "F.Cu") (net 5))
 (segment (start 225.301 90.601) (end 224.7 90) (width 0.6) (layer "F.Cu") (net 5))
 (segment (start 203.65 85.35) (end 208 85.35) (width 0.6) (layer "F.Cu") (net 5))
 (segment (start 225.101 88.899) (end 224 90) (width 0.6) (layer "F.Cu") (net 5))
 (segment (start 203.35 104.54) (end 203.753 104.54) (width 0.6) (layer "F.Cu") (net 5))
 (segment (start 203.753 104.54) (end 204.8 104.54) (width 0.6) (layer "F.Cu") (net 5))
 (segment (start 224.2 82.998) (end 225.101 83.899) (width 0.6) (layer "F.Cu") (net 5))
 (segment (start 217.201 93.201) (end 224.809424 93.201) (width 0.6) (layer "F.Cu") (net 5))
 (segment (start 208 85.35) (end 208 83.3) (width 0.6) (layer "F.Cu") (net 5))
 (segment (start 204.8 104.54) (end 209.301 100.039) (width 0.6) (layer "F.Cu") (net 5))
 (segment (start 209.301 100.039) (end 209.301 88.1766) (width 0.6) (layer "F.Cu") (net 5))
 (segment (start 216.54 111.46) (end 216.54 111.638) (width 0.6) (layer "F.Cu") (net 5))
 (segment (start 216.54 112) (end 222.54 106) (width 0.6) (layer "F.Cu") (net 5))
 (segment (start 216.54 112) (end 215.264 113.276) (width 0.6) (layer "F.Cu") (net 5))
 (segment (start 208 83.3) (end 208.302 82.998) (width 0.6) (layer "F.Cu") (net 5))
 (segment (start 205.1065 105.8935) (end 205.1065 105.9965) (width 0.25) (layer "F.Cu") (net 5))
 (segment (start 199.65 88.35) (end 200.65 88.35) (width 0.6) (layer "F.Cu") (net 5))
 (segment (start 225.101 83.899) (end 225.101 86.101) (width 0.6) (layer "F.Cu") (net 5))
 (segment (start 194.7 83.4) (end 199.65 88.35) (width 0.6) (layer "F.Cu") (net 5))
 (segment (start 200.65 88.35) (end 203.249 88.35) (width 0.6) (layer "F.Cu") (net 5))
 (segment (start 222.54 106) (end 223 106) (width 0.25) (layer "F.Cu") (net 5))
 (segment (start 216.54 112) (end 215.804537 112) (width 0.25) (layer "F.Cu") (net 5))
 (segment (start 208.302 82.998) (end 224.2 82.998) (width 0.6) (layer "F.Cu") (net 5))
 (segment (start 194.7 76) (end 194.7 83.4) (width 0.6) (layer "F.Cu") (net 5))
 (segment (start 216 92) (end 217.201 93.201) (width 0.6) (layer "F.Cu") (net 5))
 (segment (start 208.723 87.599) (end 204 87.599) (width 0.6) (layer "F.Cu") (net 5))
 (segment (start 224.7 90) (end 224 90) (width 0.6) (layer "F.Cu") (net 5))
 (segment (start 200.65 88.35) (end 203.65 85.35) (width 0.6) (layer "F.Cu") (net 5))
 (segment (start 225.301 92.709424) (end 225.301 90.601) (width 0.6) (layer "F.Cu") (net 5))
 (segment (start 209.301 88.1766) (end 208.723 87.599) (width 0.6) (layer "F.Cu") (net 5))
 (segment (start 203.249 88.35) (end 204 87.599) (width 0.6) (layer "F.Cu") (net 5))
 (segment (start 203.753 104.54) (end 205.1065 105.8935) (width 0.6) (layer "F.Cu") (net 5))
 (segment (start 216.54 112) (end 216.54 111.638) (width 0.25) (layer "F.Cu") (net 5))
 (segment (start 224.809424 93.201) (end 225.301 92.709424) (width 0.6) (layer "F.Cu") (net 5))
 (segment (start 187.7 86.9) (end 188 87.2) (width 0.6) (layer "F.Cu") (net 11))
 (segment (start 187.7 76) (end 187.7 86.9) (width 0.6) (layer "F.Cu") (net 11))
 (segment (start 217.989576 96) (end 214 92.010424) (width 0.6) (layer "F.Cu") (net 9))
 (segment (start 189 98) (end 188.3 98) (width 0.6) (layer "F.Cu") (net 9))
 (segment (start 219.08 111.92) (end 219.08 112) (width 0.6) (layer "F.Cu") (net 9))
 (segment (start 217.101 83.899) (end 213 83.899) (width 0.6) (layer "F.Cu") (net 9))
 (segment (start 188.3 98) (end 187.699 98.601) (width 0.6) (layer "F.Cu") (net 9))
 (segment (start 224.326 105.251) (end 223 103.925) (width 0.6) (layer "F.Cu") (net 9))
 (segment (start 188 97) (end 189 98) (width 0.6) (layer "F.Cu") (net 9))
 (segment (start 224 85) (end 218.202 85) (width 0.6) (layer "F.Cu") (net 9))
 (segment (start 214 87.598) (end 215.497 86.101) (width 0.6) (layer "F.Cu") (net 9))
 (segment (start 210.65 86.249) (end 210.65 100.73) (width 0.6) (layer "F.Cu") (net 9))
 (segment (start 219.08 112) (end 224.326 106.754) (width 0.6) (layer "F.Cu") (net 9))
 (segment (start 188 94) (end 188 97) (width 0.6) (layer "F.Cu") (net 9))
 (segment (start 214 92.010424) (end 214 87.598) (width 0.6) (layer "F.Cu") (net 9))
 (segment (start 187.699 113.699) (end 188.352 114.352) (width 0.6) (layer "F.Cu") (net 9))
 (segment (start 224.326 106.754) (end 224.326 105.251) (width 0.6) (layer "F.Cu") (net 9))
 (segment (start 223 96) (end 217.989576 96) (width 0.6) (layer "F.Cu") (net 9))
 (segment (start 223 103.925) (end 223 96) (width 0.6) (layer "F.Cu") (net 9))
 (segment (start 218.202 85) (end 217.101 83.899) (width 0.6) (layer "F.Cu") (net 9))
 (segment (start 188.352 114.352) (end 216.728 114.352) (width 0.6) (layer "F.Cu") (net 9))
 (segment (start 215.497 86.101) (end 222.899 86.101) (width 0.6) (layer "F.Cu") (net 9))
 (segment (start 222.899 86.101) (end 224 85) (width 0.6) (layer "F.Cu") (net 9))
 (segment (start 216.728 114.352) (end 219.08 112) (width 0.6) (layer "F.Cu") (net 9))
 (segment (start 213 83.899) (end 210.65 86.249) (width 0.6) (layer "F.Cu") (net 9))
 (segment (start 187.699 98.601) (end 187.699 113.699) (width 0.6) (layer "F.Cu") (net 9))
 (segment (start 196 90) (end 196 89.9896) (width 0.6) (layer "F.Cu") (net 12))
 (segment (start 193.291 88.699) (end 190.301 91.6886) (width 0.6) (layer "F.Cu") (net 12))
 (segment (start 190.301 99.399) (end 189.7 100) (width 0.6) (layer "F.Cu") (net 12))
 (segment (start 198 90) (end 199.65 91.65) (width 0.6) (layer "F.Cu") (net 12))
 (segment (start 196 90) (end 198 90) (width 0.6) (layer "F.Cu") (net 12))
 (segment (start 190.301 98.7094) (end 190.301 76.601) (width 0.6) (layer "F.Cu") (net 12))
 (segment (start 196 89.9896) (end 194.709 88.699) (width 0.6) (layer "F.Cu") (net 12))
 (segment (start 194.709 88.699) (end 193.291 88.699) (width 0.6) (layer "F.Cu") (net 12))
 (segment (start 190.301 76.601) (end 190.2 76.5) (width 0.6) (layer "F.Cu") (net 12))
 (segment (start 189.7 100) (end 189 100) (width 0.6) (layer "F.Cu") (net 12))
 (segment (start 190.301 91.6886) (end 190.301 99.399) (width 0.6) (layer "F.Cu") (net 12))
 (segment (start 198.927 89.401) (end 192.2 82.6744) (width 0.6) (layer "F.Cu") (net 2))
 (segment (start 208 91) (end 208 88.65) (width 0.6) (layer "F.Cu") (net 2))
 (segment (start 192.2 82.6744) (end 192.2 76.5) (width 0.6) (layer "F.Cu") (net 2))
 (segment (start 207.249 89.401) (end 198.927 89.401) (width 0.6) (layer "F.Cu") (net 2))
 (segment (start 208 88.65) (end 207.249 89.401) (width 0.6) (layer "F.Cu") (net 2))
 (segment (start 224 92) (end 223.3 92) (width 0.6) (layer "F.Cu") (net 10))
 (segment (start 223.3 92) (end 222.699 91.399) (width 0.6) (layer "F.Cu") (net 10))
 (segment (start 222.699 89.101) (end 224 87.8) (width 0.6) (layer "F.Cu") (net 10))
 (segment (start 222.699 91.399) (end 222.699 89.101) (width 0.6) (layer "F.Cu") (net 10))
 (segment (start 210.65 104.54) (end 210.65 111.19) (width 0.6) (layer "F.Cu") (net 6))
 (segment (start 210.65 111.19) (end 211.46 112) (width 0.6) (layer "F.Cu") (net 6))
 (segment (start 194 90) (end 194 94.1) (width 0.6) (layer "F.Cu") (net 4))
 (segment (start 194 94.1) (end 194 107.462) (width 0.6) (layer "F.Cu") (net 4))
 (segment (start 203.35 102) (end 204.453 102) (width 0.6) (layer "F.Cu") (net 4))
 (segment (start 205 98) (end 197.9 98) (width 0.6) (layer "F.Cu") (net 4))
 (segment (start 206.726 99.7264) (end 205 98) (width 0.6) (layer "F.Cu") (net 4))
 (segment (start 194.769 108.231) (end 194.769 112.601) (width 0.6) (layer "F.Cu") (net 4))
 (segment (start 194 90) (end 193.899 89.899) (width 0.6) (layer "F.Cu") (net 4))
 (segment (start 194.769 112.601) (end 195.619 113.451) (width 0.6) (layer "F.Cu") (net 4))
 (segment (start 204.453 102) (end 206.726 99.7264) (width 0.6) (layer "F.Cu") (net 4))
 (segment (start 195.619 113.451) (end 202.389 113.451) (width 0.6) (layer "F.Cu") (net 4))
 (segment (start 202.389 113.451) (end 203.84 112) (width 0.6) (layer "F.Cu") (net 4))
 (segment (start 197.9 98) (end 194 94.1) (width 0.6) (layer "F.Cu") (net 4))
 (segment (start 194 107.462) (end 194.769 108.231) (width 0.6) (layer "F.Cu") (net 4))
 (segment (start 210.65 102) (end 209 102) (width 0.6) (layer "F.Cu") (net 8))
 (segment (start 206.38 104.62) (end 206.38 112) (width 0.6) (layer "F.Cu") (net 8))
 (segment (start 209 102) (end 206.38 104.62) (width 0.6) (layer "F.Cu") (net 8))
 (segment (start 198.76 103.87) (end 201.9 100.73) (width 0.6) (layer "F.Cu") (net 3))
 (segment (start 201.9 100.73) (end 203.35 100.73) (width 0.6) (layer "F.Cu") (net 3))
 (segment (start 198.76 112) (end 198.76 103.87) (width 0.6) (layer "F.Cu") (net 3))
 (segment (start 208 99.727) (end 204.457 103.27) (width 0.6) (layer "F.Cu") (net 1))
 (segment (start 201.3 103.87) (end 201.3 112) (width 0.6) (layer "F.Cu") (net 1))
 (segment (start 208 93) (end 208 99.727) (width 0.6) (layer "F.Cu") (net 1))
 (segment (start 204.457 103.27) (end 203.35 103.27) (width 0.6) (layer "F.Cu") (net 1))
 (segment (start 201.9 103.27) (end 201.3 103.87) (width 0.6) (layer "F.Cu") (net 1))
 (segment (start 203.35 103.27) (end 201.9 103.27) (width 0.6) (layer "F.Cu") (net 1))
 (segment (start 209.543 103.27) (end 208.92 103.893) (width 0.6) (layer "F.Cu") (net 7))
 (segment (start 211.757 103.27) (end 210.65 103.27) (width 0.6) (layer "F.Cu") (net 7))
 (segment (start 208.92 103.893) (end 208.92 112) (width 0.6) (layer "F.Cu") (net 7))
 (segment (start 212.101 102.926) (end 211.757 103.27) (width 0.6) (layer "F.Cu") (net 7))
 (segment (start 212.101 86.899) (end 212.101 102.926) (width 0.6) (layer "F.Cu") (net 7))
 (segment (start 210.65 103.27) (end 209.543 103.27) (width 0.6) (layer "F.Cu") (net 7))
 (segment (start 216 85) (end 214 85) (width 0.6) (layer "F.Cu") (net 7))
 (segment (start 214 85) (end 212.101 86.899) (width 0.6) (layer "F.Cu") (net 7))
 (segment (start 216 90) (end 216 87.8) (width 0.6) (layer "F.Cu") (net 13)))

